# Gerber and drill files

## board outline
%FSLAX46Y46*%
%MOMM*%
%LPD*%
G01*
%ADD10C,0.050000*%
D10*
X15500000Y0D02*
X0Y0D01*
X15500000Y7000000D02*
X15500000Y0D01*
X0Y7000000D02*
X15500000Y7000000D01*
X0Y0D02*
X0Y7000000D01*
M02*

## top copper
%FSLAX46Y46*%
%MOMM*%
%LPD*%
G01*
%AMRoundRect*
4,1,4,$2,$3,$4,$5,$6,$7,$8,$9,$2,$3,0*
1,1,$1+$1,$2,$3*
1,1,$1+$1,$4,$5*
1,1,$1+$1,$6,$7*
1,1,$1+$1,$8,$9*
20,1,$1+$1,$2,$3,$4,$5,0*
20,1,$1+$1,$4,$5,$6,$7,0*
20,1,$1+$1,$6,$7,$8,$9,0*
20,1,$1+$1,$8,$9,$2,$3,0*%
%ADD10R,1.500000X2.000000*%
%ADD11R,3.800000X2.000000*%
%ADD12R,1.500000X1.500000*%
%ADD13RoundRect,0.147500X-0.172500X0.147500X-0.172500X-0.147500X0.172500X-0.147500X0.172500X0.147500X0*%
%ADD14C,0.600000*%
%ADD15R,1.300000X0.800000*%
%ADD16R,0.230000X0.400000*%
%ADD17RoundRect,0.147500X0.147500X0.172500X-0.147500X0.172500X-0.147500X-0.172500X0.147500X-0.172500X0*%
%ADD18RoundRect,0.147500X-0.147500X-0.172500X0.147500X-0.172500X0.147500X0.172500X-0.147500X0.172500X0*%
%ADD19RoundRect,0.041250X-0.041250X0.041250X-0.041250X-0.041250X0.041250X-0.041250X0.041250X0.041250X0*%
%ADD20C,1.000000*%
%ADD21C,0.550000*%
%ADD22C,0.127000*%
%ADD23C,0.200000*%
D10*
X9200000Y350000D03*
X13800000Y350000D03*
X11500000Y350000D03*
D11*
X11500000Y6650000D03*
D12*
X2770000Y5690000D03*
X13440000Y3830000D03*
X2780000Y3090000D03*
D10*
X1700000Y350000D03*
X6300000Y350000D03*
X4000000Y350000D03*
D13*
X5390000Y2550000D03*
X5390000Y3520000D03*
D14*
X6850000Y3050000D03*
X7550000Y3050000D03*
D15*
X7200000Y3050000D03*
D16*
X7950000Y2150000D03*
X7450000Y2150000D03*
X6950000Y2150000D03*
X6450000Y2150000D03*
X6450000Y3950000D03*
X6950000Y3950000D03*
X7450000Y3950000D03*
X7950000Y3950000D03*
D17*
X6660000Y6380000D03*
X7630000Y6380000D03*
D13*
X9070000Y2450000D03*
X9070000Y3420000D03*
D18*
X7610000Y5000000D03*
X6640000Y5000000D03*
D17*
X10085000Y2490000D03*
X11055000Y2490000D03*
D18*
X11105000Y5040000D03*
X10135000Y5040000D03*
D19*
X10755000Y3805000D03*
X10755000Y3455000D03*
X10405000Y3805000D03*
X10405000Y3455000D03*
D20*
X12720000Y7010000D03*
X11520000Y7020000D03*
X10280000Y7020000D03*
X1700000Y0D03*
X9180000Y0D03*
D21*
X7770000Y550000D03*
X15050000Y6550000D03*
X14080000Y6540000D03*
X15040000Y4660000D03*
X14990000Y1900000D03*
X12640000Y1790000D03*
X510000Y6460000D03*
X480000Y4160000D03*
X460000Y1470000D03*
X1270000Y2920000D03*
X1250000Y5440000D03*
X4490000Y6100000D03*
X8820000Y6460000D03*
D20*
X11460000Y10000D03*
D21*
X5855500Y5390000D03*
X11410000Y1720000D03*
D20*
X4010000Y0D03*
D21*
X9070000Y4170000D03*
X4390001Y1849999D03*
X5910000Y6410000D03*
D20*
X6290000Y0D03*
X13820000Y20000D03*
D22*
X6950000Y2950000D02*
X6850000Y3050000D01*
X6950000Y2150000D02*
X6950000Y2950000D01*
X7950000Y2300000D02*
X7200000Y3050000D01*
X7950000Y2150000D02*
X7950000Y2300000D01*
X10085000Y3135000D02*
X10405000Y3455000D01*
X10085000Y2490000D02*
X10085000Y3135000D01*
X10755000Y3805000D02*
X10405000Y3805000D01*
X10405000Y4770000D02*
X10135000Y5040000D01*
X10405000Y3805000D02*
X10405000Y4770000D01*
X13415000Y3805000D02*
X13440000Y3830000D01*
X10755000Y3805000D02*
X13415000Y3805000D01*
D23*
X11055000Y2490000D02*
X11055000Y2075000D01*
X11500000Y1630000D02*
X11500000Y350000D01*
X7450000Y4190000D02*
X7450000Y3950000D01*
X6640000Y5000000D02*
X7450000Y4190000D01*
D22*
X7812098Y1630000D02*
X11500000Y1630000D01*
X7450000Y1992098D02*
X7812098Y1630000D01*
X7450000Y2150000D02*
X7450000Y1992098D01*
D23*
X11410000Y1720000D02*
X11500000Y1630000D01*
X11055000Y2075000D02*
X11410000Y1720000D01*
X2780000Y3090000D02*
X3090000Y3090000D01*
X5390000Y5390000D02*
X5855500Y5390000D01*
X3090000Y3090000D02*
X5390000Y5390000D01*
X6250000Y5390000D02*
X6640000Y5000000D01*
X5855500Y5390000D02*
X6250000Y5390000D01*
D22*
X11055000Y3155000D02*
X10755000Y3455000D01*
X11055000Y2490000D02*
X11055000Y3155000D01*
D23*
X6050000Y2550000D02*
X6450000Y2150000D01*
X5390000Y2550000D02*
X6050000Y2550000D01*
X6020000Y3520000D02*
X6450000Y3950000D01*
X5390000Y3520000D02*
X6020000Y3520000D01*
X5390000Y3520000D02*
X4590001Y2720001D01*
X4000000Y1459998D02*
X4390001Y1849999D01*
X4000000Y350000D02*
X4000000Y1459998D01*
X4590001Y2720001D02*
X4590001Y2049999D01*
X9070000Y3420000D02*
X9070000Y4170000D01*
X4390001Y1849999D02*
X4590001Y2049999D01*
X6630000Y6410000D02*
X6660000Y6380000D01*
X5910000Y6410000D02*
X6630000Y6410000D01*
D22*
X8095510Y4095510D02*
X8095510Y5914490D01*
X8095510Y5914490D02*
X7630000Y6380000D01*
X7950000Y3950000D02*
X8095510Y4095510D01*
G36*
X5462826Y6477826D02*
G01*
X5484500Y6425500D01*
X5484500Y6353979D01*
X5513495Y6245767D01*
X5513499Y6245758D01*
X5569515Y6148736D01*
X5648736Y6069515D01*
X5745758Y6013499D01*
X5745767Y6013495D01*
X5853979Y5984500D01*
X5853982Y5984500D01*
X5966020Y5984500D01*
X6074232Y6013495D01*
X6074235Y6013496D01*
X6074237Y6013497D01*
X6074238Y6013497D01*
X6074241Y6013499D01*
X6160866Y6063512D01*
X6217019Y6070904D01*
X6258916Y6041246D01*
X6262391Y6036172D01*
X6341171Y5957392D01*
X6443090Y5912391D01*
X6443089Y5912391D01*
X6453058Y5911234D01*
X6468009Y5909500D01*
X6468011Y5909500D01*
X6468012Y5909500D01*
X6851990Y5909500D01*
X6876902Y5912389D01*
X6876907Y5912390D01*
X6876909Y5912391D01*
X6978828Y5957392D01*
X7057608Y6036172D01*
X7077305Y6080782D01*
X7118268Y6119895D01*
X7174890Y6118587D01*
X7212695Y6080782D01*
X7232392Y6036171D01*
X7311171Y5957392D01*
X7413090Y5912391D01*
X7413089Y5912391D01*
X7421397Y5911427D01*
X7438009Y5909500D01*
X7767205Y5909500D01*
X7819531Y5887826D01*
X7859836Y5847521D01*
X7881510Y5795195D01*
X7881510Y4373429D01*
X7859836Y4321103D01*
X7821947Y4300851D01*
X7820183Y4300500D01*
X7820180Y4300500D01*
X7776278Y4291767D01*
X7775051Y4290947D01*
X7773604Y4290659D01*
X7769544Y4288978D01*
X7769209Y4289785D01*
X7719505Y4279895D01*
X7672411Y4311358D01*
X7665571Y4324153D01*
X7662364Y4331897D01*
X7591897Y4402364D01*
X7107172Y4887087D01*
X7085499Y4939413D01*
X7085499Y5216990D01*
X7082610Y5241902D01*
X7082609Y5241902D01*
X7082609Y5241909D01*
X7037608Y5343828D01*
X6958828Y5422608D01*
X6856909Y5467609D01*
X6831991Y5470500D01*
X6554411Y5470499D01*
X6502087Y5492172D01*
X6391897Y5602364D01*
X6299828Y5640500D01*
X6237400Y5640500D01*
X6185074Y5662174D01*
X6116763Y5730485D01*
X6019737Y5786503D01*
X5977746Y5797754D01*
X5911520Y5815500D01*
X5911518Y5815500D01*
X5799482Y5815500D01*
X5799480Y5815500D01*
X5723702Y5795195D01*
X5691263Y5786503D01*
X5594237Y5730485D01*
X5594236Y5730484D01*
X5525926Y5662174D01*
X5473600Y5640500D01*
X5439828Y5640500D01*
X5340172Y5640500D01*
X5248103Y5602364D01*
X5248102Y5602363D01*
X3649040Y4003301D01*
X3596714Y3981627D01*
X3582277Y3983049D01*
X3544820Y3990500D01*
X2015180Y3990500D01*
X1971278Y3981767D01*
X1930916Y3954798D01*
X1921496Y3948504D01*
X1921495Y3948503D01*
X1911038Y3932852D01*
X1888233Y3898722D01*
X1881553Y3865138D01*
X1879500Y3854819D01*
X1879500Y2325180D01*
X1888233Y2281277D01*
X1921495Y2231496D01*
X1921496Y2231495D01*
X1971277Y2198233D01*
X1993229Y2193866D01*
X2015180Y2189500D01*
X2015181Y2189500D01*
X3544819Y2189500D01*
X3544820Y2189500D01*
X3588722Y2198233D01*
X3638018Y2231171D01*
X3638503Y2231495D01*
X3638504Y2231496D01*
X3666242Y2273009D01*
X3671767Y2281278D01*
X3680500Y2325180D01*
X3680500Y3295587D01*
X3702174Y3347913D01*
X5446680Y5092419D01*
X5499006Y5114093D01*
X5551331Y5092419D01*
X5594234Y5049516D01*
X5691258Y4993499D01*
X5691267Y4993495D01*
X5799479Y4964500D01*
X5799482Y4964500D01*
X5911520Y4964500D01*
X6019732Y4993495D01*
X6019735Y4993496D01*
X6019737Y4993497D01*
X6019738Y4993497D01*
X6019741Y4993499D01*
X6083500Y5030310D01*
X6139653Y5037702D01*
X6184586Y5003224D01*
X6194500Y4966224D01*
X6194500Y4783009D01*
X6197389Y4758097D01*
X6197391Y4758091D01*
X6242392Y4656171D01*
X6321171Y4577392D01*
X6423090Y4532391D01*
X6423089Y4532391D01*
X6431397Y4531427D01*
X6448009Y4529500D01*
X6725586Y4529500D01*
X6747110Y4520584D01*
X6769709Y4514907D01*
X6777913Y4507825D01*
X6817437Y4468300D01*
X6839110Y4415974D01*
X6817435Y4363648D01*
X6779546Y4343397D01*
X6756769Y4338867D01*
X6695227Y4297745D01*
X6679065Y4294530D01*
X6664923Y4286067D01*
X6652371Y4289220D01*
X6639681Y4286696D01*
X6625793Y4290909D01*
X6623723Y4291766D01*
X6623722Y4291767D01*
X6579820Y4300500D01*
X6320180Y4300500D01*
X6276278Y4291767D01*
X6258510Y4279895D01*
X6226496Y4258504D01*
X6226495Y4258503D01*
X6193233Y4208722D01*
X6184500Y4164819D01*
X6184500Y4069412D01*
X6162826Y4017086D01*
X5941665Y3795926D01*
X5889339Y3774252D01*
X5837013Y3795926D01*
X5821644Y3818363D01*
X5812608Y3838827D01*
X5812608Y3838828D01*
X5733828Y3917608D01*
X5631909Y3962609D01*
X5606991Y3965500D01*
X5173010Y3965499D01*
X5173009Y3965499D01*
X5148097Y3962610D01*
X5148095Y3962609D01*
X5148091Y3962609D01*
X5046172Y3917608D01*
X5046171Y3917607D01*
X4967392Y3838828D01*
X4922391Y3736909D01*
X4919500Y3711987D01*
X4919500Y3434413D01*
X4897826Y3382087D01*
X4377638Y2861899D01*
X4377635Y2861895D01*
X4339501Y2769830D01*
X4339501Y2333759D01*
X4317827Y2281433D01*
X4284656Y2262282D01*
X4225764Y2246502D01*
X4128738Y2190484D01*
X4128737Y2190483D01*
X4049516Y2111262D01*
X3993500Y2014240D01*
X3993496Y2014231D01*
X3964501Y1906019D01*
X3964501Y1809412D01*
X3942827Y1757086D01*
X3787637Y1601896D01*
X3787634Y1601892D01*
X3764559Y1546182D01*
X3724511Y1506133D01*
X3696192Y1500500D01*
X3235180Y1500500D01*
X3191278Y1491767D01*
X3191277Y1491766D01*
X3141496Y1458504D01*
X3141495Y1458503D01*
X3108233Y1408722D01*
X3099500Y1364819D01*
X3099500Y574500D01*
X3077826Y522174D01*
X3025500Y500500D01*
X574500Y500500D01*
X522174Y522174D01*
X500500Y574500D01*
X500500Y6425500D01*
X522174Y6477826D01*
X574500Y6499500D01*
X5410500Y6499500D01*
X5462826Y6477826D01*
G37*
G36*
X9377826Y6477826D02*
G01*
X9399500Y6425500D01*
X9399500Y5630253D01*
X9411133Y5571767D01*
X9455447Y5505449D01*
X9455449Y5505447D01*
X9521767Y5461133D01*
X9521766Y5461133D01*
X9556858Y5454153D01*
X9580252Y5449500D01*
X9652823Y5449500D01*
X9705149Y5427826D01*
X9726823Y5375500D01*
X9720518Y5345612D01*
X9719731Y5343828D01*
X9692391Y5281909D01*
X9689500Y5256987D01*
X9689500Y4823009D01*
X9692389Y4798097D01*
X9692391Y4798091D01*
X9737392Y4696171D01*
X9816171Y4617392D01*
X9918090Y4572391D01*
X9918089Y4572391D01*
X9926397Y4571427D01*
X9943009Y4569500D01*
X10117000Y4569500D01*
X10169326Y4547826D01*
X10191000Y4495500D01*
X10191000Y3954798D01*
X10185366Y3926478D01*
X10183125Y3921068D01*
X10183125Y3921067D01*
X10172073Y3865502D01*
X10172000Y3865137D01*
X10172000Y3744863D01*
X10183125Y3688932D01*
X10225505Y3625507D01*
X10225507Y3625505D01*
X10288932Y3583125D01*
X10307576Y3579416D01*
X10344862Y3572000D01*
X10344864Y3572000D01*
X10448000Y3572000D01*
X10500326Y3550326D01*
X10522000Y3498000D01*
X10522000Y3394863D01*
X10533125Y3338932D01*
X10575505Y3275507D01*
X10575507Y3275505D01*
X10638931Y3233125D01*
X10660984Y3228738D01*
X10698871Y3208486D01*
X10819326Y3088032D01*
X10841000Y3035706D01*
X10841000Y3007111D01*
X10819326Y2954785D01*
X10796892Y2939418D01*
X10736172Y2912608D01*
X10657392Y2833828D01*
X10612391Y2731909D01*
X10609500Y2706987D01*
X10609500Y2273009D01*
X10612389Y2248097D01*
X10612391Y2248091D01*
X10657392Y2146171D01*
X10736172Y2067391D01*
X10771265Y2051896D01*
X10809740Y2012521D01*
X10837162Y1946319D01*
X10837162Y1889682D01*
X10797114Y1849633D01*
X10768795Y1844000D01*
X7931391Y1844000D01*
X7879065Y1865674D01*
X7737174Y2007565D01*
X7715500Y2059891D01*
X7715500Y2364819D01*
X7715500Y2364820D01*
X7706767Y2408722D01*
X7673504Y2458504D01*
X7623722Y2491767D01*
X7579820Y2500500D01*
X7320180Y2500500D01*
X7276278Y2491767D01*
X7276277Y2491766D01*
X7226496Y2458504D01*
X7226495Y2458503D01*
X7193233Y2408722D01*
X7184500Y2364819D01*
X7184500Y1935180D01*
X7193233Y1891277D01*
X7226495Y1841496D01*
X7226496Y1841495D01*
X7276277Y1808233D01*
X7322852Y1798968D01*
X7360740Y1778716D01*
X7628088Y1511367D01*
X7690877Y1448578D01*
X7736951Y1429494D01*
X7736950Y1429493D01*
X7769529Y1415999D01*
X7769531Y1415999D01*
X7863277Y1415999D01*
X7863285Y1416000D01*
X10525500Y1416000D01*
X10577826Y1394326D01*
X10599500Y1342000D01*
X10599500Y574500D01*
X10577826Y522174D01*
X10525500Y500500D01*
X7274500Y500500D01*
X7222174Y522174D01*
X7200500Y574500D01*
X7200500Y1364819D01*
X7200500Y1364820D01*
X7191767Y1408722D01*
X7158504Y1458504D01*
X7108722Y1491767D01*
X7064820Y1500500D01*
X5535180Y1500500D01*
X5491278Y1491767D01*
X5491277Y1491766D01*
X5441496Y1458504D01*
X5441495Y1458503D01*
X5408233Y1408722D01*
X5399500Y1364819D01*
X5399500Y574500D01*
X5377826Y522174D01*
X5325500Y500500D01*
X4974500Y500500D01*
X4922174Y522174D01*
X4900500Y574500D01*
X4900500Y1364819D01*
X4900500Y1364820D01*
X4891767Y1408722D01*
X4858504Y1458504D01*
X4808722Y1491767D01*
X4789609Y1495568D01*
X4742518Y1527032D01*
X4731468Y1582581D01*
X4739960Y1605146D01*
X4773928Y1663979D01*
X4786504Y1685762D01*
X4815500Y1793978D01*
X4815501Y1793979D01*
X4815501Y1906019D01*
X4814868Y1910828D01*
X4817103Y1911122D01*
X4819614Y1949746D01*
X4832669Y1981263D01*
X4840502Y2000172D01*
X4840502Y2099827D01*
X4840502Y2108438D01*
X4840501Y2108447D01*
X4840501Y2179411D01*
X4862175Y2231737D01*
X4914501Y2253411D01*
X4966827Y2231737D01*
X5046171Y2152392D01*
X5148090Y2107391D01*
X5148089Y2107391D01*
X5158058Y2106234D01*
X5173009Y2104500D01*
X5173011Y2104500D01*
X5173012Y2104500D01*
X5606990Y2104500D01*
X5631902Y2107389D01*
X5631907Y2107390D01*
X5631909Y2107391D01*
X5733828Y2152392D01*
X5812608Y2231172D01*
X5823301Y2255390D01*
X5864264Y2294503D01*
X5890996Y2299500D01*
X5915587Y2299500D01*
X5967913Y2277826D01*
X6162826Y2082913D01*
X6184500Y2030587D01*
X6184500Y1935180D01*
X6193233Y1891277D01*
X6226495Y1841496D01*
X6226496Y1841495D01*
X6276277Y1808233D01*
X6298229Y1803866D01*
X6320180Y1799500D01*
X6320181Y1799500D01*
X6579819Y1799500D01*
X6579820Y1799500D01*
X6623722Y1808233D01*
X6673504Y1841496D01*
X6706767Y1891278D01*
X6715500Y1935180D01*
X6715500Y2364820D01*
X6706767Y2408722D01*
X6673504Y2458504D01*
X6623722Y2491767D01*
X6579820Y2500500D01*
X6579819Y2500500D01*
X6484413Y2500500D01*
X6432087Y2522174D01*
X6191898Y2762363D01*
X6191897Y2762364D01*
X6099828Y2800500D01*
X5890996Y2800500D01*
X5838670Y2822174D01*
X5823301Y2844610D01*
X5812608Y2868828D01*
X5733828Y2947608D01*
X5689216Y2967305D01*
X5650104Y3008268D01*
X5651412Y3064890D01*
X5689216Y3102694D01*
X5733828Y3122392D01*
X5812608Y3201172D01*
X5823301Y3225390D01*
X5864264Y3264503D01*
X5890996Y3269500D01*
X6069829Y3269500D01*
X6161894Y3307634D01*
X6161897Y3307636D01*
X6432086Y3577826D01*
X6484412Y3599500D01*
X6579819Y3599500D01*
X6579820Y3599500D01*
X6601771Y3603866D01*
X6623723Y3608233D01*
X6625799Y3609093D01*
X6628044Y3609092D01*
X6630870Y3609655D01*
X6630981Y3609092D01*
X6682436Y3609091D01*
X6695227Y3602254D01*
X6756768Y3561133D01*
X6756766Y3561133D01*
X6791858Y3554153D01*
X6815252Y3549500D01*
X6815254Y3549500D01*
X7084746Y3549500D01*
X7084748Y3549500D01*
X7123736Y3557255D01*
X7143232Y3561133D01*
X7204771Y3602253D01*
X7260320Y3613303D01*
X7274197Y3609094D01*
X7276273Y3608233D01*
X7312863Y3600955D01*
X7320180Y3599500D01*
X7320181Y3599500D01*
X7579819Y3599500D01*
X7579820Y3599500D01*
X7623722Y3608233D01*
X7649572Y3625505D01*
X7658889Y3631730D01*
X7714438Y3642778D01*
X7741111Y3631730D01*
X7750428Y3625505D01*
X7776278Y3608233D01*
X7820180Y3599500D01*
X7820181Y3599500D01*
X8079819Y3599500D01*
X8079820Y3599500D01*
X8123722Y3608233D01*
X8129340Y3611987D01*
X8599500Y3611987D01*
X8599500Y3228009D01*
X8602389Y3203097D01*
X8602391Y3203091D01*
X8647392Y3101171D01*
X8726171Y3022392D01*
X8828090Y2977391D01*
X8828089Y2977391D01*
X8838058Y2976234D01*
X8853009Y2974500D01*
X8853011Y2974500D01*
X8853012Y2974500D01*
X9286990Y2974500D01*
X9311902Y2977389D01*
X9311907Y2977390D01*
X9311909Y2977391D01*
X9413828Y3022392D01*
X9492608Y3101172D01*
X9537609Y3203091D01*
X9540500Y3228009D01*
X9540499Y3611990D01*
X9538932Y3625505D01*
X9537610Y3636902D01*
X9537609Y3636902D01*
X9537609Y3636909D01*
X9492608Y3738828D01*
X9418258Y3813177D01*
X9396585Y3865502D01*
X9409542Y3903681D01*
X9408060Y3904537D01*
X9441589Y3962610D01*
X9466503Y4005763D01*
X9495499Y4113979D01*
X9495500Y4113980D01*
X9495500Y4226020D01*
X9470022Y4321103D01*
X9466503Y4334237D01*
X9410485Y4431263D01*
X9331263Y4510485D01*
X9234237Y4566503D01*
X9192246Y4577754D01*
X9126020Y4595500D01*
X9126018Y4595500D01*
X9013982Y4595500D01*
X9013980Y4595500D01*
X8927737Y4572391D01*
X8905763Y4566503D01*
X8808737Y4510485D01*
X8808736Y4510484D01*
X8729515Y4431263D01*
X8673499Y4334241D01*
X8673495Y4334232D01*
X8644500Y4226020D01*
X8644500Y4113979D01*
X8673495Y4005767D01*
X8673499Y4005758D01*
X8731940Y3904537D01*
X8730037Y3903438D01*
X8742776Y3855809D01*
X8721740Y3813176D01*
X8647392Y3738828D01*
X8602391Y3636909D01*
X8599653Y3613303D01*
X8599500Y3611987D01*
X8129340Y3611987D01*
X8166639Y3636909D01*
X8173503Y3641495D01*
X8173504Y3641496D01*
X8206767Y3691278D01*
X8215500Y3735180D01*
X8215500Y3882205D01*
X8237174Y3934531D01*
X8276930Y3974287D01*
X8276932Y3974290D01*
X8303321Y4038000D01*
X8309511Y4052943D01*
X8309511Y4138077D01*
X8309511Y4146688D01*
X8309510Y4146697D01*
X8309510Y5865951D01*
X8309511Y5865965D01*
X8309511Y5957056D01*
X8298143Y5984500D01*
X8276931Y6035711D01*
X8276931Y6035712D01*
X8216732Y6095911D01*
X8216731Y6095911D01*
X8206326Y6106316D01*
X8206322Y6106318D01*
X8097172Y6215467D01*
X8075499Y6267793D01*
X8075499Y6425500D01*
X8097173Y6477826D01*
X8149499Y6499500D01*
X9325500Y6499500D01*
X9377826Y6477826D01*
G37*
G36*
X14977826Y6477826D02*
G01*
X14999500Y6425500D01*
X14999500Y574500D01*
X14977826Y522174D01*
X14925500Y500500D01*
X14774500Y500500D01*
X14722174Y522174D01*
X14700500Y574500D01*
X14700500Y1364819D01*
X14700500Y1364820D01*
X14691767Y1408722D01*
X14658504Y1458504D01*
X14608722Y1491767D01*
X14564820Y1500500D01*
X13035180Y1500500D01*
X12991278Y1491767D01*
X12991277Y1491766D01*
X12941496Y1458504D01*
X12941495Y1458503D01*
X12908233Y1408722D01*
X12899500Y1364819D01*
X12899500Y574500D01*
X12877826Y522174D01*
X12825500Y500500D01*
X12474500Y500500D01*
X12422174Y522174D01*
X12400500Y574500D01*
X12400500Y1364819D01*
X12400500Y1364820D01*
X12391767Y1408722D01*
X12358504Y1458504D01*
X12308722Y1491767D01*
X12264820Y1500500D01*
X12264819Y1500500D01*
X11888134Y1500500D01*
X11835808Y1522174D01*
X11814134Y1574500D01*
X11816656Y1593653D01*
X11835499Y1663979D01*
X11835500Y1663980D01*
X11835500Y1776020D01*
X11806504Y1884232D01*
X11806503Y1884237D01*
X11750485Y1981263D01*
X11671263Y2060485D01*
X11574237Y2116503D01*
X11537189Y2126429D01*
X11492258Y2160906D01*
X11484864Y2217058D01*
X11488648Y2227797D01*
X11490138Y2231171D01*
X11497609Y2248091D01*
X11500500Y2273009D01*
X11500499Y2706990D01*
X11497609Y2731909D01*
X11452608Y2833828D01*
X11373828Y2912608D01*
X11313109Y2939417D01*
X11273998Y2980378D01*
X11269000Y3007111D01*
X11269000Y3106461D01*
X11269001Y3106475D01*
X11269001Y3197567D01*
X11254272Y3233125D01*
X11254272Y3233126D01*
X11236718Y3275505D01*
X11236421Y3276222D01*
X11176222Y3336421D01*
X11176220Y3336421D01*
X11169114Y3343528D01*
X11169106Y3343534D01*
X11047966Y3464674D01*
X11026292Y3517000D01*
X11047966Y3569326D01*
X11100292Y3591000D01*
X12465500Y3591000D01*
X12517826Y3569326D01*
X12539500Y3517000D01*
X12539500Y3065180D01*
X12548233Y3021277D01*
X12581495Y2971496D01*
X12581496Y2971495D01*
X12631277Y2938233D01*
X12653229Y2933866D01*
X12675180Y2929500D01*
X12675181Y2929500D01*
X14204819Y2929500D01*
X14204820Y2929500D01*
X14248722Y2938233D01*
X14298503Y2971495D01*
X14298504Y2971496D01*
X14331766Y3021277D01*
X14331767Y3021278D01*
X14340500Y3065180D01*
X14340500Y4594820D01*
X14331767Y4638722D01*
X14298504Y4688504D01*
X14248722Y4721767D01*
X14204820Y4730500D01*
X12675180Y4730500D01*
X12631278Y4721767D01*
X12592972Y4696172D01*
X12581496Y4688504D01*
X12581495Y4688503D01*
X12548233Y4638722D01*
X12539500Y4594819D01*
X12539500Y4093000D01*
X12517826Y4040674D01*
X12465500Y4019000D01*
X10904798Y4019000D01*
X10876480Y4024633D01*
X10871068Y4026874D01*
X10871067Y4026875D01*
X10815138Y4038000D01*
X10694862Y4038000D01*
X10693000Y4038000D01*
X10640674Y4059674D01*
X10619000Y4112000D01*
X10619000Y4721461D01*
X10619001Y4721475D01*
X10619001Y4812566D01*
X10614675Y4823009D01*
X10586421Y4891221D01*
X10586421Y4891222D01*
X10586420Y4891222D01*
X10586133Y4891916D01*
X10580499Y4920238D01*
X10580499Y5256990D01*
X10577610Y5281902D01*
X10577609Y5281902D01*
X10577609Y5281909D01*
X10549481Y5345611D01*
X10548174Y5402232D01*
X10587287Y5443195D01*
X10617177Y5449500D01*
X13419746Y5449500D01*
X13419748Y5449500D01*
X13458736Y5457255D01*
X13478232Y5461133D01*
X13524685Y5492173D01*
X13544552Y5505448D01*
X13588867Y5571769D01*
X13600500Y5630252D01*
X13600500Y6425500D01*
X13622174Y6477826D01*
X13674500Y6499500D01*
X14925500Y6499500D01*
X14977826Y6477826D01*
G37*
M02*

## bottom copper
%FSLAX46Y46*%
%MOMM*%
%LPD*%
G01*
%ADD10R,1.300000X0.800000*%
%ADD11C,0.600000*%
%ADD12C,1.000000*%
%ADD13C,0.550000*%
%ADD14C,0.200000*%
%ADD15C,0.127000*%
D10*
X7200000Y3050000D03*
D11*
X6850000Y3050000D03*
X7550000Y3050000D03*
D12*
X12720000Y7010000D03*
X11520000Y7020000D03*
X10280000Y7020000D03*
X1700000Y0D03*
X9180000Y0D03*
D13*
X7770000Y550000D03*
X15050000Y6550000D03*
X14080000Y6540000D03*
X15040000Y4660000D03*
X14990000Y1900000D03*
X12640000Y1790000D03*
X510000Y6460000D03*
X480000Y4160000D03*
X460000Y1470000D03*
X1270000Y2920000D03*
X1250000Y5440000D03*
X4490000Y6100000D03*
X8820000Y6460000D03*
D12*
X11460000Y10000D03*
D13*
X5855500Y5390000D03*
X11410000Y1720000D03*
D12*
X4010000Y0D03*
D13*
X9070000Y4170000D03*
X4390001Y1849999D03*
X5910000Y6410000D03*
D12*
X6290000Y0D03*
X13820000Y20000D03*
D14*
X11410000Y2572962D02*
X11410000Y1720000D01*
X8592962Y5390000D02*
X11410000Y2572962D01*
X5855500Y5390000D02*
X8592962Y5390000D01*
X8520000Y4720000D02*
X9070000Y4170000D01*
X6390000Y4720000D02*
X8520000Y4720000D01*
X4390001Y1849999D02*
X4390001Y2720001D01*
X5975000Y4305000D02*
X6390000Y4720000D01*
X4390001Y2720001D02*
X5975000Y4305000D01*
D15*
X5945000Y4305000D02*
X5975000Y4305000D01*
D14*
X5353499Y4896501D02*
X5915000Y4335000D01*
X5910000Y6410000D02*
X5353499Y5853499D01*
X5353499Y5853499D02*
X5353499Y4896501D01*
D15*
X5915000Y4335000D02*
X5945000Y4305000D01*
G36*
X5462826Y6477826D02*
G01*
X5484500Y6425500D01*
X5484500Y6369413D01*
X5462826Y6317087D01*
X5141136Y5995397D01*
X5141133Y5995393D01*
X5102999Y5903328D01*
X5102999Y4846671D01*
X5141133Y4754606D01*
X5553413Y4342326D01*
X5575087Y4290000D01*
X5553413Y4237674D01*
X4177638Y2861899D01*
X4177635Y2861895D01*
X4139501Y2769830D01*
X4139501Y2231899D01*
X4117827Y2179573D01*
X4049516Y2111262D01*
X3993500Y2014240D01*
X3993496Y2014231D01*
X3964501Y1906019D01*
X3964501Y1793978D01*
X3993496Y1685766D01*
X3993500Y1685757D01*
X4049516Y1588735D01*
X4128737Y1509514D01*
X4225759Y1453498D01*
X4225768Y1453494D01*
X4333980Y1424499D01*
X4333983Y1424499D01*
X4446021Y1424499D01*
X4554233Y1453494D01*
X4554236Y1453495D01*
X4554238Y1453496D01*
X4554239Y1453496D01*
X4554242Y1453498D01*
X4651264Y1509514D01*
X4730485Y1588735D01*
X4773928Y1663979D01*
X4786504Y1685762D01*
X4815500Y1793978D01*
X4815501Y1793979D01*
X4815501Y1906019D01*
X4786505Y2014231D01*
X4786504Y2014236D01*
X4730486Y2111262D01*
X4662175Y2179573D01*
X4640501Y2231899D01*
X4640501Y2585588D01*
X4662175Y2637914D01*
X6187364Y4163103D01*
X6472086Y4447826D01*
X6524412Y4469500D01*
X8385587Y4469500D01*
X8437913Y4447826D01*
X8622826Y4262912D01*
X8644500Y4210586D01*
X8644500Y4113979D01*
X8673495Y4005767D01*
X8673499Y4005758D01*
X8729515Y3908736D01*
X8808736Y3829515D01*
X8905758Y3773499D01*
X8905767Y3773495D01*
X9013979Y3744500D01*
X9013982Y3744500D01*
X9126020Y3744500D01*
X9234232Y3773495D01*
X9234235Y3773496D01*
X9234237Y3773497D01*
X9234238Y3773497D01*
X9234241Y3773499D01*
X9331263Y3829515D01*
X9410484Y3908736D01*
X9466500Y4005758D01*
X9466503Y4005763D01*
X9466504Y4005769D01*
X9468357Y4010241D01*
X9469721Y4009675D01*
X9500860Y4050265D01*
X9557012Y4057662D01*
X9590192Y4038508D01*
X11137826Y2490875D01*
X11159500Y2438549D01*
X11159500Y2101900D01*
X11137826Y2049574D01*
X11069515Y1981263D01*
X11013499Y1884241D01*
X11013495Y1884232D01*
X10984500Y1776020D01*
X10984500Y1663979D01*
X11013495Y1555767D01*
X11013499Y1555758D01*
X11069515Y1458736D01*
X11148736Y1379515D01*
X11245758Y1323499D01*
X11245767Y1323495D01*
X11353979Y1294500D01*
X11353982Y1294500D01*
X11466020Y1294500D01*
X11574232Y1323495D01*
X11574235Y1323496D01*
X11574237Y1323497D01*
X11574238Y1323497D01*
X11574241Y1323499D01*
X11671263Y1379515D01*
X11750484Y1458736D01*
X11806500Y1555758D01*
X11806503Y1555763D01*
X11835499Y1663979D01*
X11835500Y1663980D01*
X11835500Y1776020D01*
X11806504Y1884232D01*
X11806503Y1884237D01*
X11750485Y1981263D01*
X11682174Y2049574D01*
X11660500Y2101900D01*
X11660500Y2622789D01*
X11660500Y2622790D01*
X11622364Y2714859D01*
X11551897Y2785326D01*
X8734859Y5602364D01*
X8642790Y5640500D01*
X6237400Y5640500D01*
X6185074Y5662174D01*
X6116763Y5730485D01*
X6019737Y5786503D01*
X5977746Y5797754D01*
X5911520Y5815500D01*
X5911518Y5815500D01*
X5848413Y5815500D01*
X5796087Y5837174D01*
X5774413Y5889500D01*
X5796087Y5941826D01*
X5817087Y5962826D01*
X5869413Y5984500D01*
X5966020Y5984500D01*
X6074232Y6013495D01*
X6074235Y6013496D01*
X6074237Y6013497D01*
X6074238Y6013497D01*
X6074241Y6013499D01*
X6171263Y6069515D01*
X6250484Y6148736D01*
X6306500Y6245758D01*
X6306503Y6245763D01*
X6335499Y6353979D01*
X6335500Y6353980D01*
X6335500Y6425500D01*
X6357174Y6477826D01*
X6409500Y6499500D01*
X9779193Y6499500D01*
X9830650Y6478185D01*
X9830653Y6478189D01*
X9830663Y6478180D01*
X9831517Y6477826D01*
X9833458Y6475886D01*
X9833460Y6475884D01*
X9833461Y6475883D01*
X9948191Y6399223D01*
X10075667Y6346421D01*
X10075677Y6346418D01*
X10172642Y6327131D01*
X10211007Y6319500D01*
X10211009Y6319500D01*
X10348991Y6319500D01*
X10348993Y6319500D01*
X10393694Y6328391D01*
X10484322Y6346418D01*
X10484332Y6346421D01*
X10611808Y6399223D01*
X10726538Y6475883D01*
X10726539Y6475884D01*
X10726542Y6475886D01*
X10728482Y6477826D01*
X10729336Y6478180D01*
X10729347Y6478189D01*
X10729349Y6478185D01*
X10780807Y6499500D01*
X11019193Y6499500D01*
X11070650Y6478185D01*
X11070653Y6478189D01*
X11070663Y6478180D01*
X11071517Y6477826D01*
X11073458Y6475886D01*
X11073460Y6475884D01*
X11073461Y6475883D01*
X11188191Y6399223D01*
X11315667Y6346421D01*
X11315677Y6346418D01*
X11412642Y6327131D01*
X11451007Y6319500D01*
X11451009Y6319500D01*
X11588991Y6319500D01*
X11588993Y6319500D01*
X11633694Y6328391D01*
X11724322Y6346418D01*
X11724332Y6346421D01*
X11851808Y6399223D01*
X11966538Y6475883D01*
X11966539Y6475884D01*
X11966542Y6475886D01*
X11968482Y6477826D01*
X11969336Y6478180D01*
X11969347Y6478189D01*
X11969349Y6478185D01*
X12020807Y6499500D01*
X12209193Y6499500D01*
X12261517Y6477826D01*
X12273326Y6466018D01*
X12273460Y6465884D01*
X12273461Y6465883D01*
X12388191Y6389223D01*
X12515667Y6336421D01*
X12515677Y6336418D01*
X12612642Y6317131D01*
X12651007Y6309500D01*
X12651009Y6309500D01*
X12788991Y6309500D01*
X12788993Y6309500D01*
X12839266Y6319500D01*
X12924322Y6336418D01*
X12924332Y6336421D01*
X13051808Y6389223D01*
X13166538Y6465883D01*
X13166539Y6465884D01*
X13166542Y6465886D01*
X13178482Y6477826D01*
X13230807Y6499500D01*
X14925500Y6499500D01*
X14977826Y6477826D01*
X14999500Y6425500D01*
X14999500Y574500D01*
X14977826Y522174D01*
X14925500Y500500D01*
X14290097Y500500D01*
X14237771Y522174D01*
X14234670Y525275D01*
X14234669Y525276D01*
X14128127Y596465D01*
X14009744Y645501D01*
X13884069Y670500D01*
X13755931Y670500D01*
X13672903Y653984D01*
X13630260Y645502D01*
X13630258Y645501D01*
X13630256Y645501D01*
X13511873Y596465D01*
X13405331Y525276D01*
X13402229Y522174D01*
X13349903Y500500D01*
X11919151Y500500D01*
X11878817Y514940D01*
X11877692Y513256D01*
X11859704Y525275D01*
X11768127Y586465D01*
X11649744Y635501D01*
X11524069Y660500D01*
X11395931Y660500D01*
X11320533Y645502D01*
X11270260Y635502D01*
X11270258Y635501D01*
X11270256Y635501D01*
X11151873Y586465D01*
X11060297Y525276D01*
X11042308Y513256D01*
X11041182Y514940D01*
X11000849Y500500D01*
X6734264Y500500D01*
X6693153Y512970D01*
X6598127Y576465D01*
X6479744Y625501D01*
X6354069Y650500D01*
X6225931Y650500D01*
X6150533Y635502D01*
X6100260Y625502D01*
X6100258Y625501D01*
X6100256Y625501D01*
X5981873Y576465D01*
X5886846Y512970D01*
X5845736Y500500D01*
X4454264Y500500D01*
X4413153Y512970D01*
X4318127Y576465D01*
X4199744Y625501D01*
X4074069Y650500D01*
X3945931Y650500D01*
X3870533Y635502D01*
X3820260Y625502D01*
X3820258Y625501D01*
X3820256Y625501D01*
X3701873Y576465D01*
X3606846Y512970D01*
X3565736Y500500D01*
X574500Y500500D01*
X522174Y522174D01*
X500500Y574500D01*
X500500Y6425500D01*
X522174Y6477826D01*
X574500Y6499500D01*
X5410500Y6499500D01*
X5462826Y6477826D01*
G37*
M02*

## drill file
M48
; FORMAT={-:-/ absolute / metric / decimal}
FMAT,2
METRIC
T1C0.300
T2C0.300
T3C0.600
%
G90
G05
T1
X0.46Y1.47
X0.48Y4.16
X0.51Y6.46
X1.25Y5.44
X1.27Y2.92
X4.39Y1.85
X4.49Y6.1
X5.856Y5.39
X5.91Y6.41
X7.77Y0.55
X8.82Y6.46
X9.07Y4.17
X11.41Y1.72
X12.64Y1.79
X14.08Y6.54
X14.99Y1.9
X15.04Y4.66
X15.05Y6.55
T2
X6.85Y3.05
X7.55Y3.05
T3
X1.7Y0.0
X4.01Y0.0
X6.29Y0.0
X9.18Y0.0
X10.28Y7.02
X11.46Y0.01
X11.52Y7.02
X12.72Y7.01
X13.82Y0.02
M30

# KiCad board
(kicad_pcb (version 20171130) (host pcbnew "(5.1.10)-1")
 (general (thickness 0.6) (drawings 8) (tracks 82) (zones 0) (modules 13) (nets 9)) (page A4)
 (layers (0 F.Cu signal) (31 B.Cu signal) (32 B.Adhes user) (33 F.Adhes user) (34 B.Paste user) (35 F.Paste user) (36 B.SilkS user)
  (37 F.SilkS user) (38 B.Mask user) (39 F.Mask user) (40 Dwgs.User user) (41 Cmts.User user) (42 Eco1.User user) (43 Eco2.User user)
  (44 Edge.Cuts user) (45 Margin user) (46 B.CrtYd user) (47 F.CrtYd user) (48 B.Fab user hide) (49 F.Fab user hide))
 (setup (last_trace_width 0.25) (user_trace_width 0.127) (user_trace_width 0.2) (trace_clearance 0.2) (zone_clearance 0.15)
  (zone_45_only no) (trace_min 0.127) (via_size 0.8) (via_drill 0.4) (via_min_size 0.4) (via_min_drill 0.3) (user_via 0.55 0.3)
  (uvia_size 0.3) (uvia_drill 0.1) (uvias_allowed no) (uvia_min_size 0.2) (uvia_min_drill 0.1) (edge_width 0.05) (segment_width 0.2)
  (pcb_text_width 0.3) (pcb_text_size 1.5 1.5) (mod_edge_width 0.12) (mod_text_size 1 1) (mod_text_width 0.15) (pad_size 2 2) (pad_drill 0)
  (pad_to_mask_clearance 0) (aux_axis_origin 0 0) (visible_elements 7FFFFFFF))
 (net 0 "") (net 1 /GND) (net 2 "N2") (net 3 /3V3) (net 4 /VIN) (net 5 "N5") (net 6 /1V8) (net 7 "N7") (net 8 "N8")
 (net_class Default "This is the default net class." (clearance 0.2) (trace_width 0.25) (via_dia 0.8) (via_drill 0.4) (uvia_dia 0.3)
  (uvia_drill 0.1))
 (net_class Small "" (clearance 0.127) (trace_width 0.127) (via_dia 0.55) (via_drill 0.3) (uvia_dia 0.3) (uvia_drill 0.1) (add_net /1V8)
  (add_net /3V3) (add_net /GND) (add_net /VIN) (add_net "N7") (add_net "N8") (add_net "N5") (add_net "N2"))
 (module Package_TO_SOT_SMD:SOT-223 (layer F.Cu) (at 11.5 -3.5 90)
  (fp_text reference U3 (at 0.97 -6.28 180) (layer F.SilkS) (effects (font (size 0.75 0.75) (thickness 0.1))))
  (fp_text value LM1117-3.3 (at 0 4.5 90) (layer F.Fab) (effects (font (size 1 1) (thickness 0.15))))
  (pad 1 smd rect (at -3.15 -2.3 90) (size 2 1.5) (layers F.Cu F.Paste F.Mask) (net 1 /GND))
  (pad 3 smd rect (at -3.15 2.3 90) (size 2 1.5) (layers F.Cu F.Paste F.Mask) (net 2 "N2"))
  (pad 2 smd rect (at -3.15 0 90) (size 2 1.5) (layers F.Cu F.Paste F.Mask) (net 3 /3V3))
  (pad 4 smd rect (at 3.15 0 90) (size 2 3.8) (layers F.Cu F.Paste F.Mask)))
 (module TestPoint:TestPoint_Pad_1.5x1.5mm (layer F.Cu) (at 2.77 -5.69)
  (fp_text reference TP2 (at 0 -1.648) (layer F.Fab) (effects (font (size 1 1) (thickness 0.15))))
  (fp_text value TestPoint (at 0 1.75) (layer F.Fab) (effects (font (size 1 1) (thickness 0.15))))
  (pad 1 smd rect (at 0 0) (size 1.5 1.5) (layers F.Cu F.Mask) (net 1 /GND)))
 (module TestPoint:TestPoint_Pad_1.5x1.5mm (layer F.Cu) (at 13.44 -3.83)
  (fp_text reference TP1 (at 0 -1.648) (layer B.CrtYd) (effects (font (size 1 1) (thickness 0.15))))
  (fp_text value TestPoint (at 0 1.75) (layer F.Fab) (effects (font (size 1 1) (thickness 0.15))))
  (pad 1 smd rect (at 0 0) (size 1.5 1.5) (layers F.Cu F.Mask) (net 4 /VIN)))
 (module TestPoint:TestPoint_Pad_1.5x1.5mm (layer F.Cu) (at 2.78 -3.09)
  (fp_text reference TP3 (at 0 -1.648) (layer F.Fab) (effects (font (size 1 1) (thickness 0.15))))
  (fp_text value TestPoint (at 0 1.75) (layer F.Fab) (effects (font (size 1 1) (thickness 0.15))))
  (pad 1 smd rect (at 0 0) (size 1.5 1.5) (layers F.Cu F.Mask) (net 3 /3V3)))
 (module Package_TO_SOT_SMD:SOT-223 (layer F.Cu) (at 4 -3.5 90)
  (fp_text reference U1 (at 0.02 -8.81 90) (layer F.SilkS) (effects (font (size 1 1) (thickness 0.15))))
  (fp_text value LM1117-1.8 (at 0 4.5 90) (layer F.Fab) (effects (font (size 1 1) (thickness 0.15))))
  (pad 1 smd rect (at -3.15 -2.3 90) (size 2 1.5) (layers F.Cu F.Paste F.Mask) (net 1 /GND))
  (pad 3 smd rect (at -3.15 2.3 90) (size 2 1.5) (layers F.Cu F.Paste F.Mask) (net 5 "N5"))
  (pad 2 smd rect (at -3.15 0 90) (size 2 1.5) (layers F.Cu F.Paste F.Mask) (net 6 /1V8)))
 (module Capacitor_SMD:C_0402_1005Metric (layer F.Cu) (at 5.39 -3.035 270)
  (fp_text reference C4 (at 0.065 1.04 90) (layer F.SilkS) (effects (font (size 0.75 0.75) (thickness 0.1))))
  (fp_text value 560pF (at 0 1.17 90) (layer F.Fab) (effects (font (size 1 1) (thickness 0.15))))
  (pad 2 smd roundrect (at 0.485 0 270) (size 0.59 0.64) (layers F.Cu F.Paste F.Mask) (roundrect_rratio 0.25) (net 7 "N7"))
  (pad 1 smd roundrect (at -0.485 0 270) (size 0.59 0.64) (layers F.Cu F.Paste F.Mask) (roundrect_rratio 0.25) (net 6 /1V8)))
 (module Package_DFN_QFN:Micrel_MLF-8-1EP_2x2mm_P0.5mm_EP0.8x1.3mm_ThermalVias (layer F.Cu) (at 7.2 -3.05 270)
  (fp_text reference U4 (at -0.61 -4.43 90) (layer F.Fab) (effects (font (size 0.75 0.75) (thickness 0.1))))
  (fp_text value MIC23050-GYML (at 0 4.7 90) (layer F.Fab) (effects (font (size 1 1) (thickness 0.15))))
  (pad 9 smd rect (at 0 0 270) (size 0.8 1.3) (layers B.Cu) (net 1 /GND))
  (pad "" smd rect (at 0 0.35 270) (size 0.55 0.55) (layers F.Paste))
  (pad "" smd rect (at 0 -0.35 270) (size 0.55 0.55) (layers F.Paste))
  (pad 9 thru_hole circle (at 0 0.35 270) (size 0.6 0.6) (drill 0.3) (layers *.Cu) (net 1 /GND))
  (pad 9 thru_hole circle (at 0 -0.35 270) (size 0.6 0.6) (drill 0.3) (layers *.Cu) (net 1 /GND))
  (pad 9 smd rect (at 0 0 270) (size 0.8 1.3) (layers F.Cu F.Mask) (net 1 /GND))
  (pad 8 smd rect (at 0.9 -0.75 270) (size 0.4 0.23) (layers F.Cu F.Paste F.Mask) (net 1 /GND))
  (pad 7 smd rect (at 0.9 -0.25 270) (size 0.4 0.23) (layers F.Cu F.Paste F.Mask) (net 3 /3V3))
  (pad 6 smd rect (at 0.9 0.25 270) (size 0.4 0.23) (layers F.Cu F.Paste F.Mask) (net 1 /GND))
  (pad 5 smd rect (at 0.9 0.75 270) (size 0.4 0.23) (layers F.Cu F.Paste F.Mask) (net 7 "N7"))
  (pad 4 smd rect (at -0.9 0.75 270) (size 0.4 0.23) (layers F.Cu F.Paste F.Mask) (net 6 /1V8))
  (pad 3 smd rect (at -0.9 0.25 270) (size 0.4 0.23) (layers F.Cu F.Paste F.Mask))
  (pad 2 smd rect (at -0.9 -0.25 270) (size 0.4 0.23) (layers F.Cu F.Paste F.Mask) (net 3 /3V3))
  (pad 1 smd rect (at -0.9 -0.75 270) (size 0.4 0.23) (layers F.Cu F.Paste F.Mask) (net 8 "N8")))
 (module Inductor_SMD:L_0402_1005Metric (layer F.Cu) (at 7.145 -6.38 180)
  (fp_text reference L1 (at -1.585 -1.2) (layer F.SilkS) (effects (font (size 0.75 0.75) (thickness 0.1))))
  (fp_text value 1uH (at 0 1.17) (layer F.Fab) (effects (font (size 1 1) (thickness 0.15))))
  (pad 2 smd roundrect (at 0.485 0 180) (size 0.59 0.64) (layers F.Cu F.Paste F.Mask) (roundrect_rratio 0.25) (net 6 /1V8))
  (pad 1 smd roundrect (at -0.485 0 180) (size 0.59 0.64) (layers F.Cu F.Paste F.Mask) (roundrect_rratio 0.25) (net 8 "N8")))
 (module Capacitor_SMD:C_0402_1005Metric (layer F.Cu) (at 9.07 -2.935 270)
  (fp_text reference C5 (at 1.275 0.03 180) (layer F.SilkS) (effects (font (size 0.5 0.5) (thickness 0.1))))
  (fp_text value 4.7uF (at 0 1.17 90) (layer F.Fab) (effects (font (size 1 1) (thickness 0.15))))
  (pad 2 smd roundrect (at 0.485 0 270) (size 0.59 0.64) (layers F.Cu F.Paste F.Mask) (roundrect_rratio 0.25) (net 1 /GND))
  (pad 1 smd roundrect (at -0.485 0 270) (size 0.59 0.64) (layers F.Cu F.Paste F.Mask) (roundrect_rratio 0.25) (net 6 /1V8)))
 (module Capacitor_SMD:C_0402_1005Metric (layer F.Cu) (at 7.125 -5)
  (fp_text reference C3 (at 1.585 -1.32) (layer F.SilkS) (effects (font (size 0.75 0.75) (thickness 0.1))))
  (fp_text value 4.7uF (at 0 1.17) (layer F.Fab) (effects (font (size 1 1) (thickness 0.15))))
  (pad 2 smd roundrect (at 0.485 0) (size 0.59 0.64) (layers F.Cu F.Paste F.Mask) (roundrect_rratio 0.25) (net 1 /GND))
  (pad 1 smd roundrect (at -0.485 0) (size 0.59 0.64) (layers F.Cu F.Paste F.Mask) (roundrect_rratio 0.25) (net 3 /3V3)))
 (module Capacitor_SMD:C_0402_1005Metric (layer F.Cu) (at 10.57 -2.49 180)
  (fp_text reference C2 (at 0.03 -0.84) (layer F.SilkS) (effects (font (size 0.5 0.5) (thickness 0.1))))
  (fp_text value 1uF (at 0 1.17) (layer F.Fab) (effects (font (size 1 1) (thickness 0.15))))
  (pad 2 smd roundrect (at 0.485 0 180) (size 0.59 0.64) (layers F.Cu F.Paste F.Mask) (roundrect_rratio 0.25) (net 1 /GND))
  (pad 1 smd roundrect (at -0.485 0 180) (size 0.59 0.64) (layers F.Cu F.Paste F.Mask) (roundrect_rratio 0.25) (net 3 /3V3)))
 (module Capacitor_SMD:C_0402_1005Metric (layer F.Cu) (at 10.62 -5.04)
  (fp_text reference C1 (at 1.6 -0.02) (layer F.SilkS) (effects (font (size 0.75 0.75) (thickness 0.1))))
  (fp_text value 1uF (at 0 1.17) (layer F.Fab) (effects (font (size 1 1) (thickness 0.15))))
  (pad 2 smd roundrect (at 0.485 0) (size 0.59 0.64) (layers F.Cu F.Paste F.Mask) (roundrect_rratio 0.25) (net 1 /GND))
  (pad 1 smd roundrect (at -0.485 0) (size 0.59 0.64) (layers F.Cu F.Paste F.Mask) (roundrect_rratio 0.25) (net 4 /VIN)))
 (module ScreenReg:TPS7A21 (layer F.Cu) (at 10.58 -3.63 270)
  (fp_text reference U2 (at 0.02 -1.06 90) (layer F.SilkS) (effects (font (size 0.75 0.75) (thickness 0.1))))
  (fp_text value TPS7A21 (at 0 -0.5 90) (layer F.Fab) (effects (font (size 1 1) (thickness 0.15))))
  (pad A1 smd roundrect (at -0.175 -0.175 270) (size 0.165 0.165) (layers F.Cu F.Paste F.Mask) (roundrect_rratio 0.25) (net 4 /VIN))
  (pad A2 smd roundrect (at 0.175 -0.175 270) (size 0.165 0.165) (layers F.Cu F.Paste F.Mask) (roundrect_rratio 0.25) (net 3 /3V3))
  (pad B1 smd roundrect (at -0.175 0.175 270) (size 0.165 0.165) (layers F.Cu F.Paste F.Mask) (roundrect_rratio 0.25) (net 4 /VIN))
  (pad B2 smd roundrect (at 0.175 0.175 270) (size 0.165 0.165) (layers F.Cu F.Paste F.Mask) (roundrect_rratio 0.25) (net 1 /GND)))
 (gr_line (start 15.5 0) (end 0 0) (layer Edge.Cuts) (width 0.05))
 (gr_line (start 15.5 -7) (end 15.5 0) (layer Edge.Cuts) (width 0.05))
 (gr_line (start 0 -7) (end 15.5 -7) (layer Edge.Cuts) (width 0.05))
 (gr_line (start 0 0) (end 0 -7) (layer Edge.Cuts) (width 0.05))
 (via (at 12.72 -7.01) (size 1) (drill 0.6) (layers F.Cu B.Cu) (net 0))
 (via (at 11.52 -7.02) (size 1) (drill 0.6) (layers F.Cu B.Cu) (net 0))
 (via (at 10.28 -7.02) (size 1) (drill 0.6) (layers F.Cu B.Cu) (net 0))
 (via (at 1.7 0) (size 1) (drill 0.6) (layers F.Cu B.Cu) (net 1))
 (via (at 9.18 0) (size 1) (drill 0.6) (layers F.Cu B.Cu) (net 1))
 (via (at 7.77 -0.55) (size 0.55) (drill 0.3) (layers F.Cu B.Cu) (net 1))
 (segment (start 6.95 -2.95) (end 6.85 -3.05) (width 0.127) (layer F.Cu) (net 1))
 (segment (start 6.95 -2.15) (end 6.95 -2.95) (width 0.127) (layer F.Cu) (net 1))
 (segment (start 7.95 -2.3) (end 7.2 -3.05) (width 0.127) (layer F.Cu) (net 1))
 (segment (start 7.95 -2.15) (end 7.95 -2.3) (width 0.127) (layer F.Cu) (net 1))
 (via (at 15.05 -6.55) (size 0.55) (drill 0.3) (layers F.Cu B.Cu) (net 1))
 (via (at 14.08 -6.54) (size 0.55) (drill 0.3) (layers F.Cu B.Cu) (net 1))
 (via (at 15.04 -4.66) (size 0.55) (drill 0.3) (layers F.Cu B.Cu) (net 1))
 (via (at 14.99 -1.9) (size 0.55) (drill 0.3) (layers F.Cu B.Cu) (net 1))
 (via (at 12.64 -1.79) (size 0.55) (drill 0.3) (layers F.Cu B.Cu) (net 1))
 (via (at 0.51 -6.46) (size 0.55) (drill 0.3) (layers F.Cu B.Cu) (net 1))
 (via (at 0.48 -4.16) (size 0.55) (drill 0.3) (layers F.Cu B.Cu) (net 1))
 (via (at 0.46 -1.47) (size 0.55) (drill 0.3) (layers F.Cu B.Cu) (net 1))
 (via (at 1.27 -2.92) (size 0.55) (drill 0.3) (layers F.Cu B.Cu) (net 1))
 (via (at 1.25 -5.44) (size 0.55) (drill 0.3) (layers F.Cu B.Cu) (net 1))
 (via (at 4.49 -6.1) (size 0.55) (drill 0.3) (layers F.Cu B.Cu) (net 1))
 (via (at 8.82 -6.46) (size 0.55) (drill 0.3) (layers F.Cu B.Cu) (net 1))
 (segment (start 10.085 -3.135) (end 10.405 -3.455) (width 0.127) (layer F.Cu) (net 1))
 (segment (start 10.085 -2.49) (end 10.085 -3.135) (width 0.127) (layer F.Cu) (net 1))
 (segment (start 10.755 -3.805) (end 10.405 -3.805) (width 0.127) (layer F.Cu) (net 4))
 (segment (start 10.405 -4.77) (end 10.135 -5.04) (width 0.127) (layer F.Cu) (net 4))
 (segment (start 10.405 -3.805) (end 10.405 -4.77) (width 0.127) (layer F.Cu) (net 4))
 (segment (start 13.415 -3.805) (end 13.44 -3.83) (width 0.127) (layer F.Cu) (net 4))
 (segment (start 10.755 -3.805) (end 13.415 -3.805) (width 0.127) (layer F.Cu) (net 4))
 (via (at 11.46 -0.01) (size 1) (drill 0.6) (layers F.Cu B.Cu) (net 3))
 (segment (start 11.055 -2.49) (end 11.055 -2.075) (width 0.2) (layer F.Cu) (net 3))
 (segment (start 11.5 -1.63) (end 11.5 -0.35) (width 0.2) (layer F.Cu) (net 3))
 (segment (start 7.45 -4.19) (end 7.45 -3.95) (width 0.2) (layer F.Cu) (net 3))
 (segment (start 6.64 -5) (end 7.45 -4.19) (width 0.2) (layer F.Cu) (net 3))
 (segment (start 7.812098 -1.63) (end 11.5 -1.63) (width 0.127) (layer F.Cu) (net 3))
 (segment (start 7.45 -1.992098) (end 7.812098 -1.63) (width 0.127) (layer F.Cu) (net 3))
 (segment (start 7.45 -2.15) (end 7.45 -1.992098) (width 0.127) (layer F.Cu) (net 3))
 (via (at 5.8555 -5.39) (size 0.55) (drill 0.3) (layers F.Cu B.Cu) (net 3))
 (via (at 11.41 -1.72) (size 0.55) (drill 0.3) (layers F.Cu B.Cu) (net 3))
 (segment (start 11.41 -1.72) (end 11.5 -1.63) (width 0.2) (layer F.Cu) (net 3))
 (segment (start 11.055 -2.075) (end 11.41 -1.72) (width 0.2) (layer F.Cu) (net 3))
 (segment (start 2.78 -3.09) (end 3.09 -3.09) (width 0.2) (layer F.Cu) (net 3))
 (segment (start 5.39 -5.39) (end 5.8555 -5.39) (width 0.2) (layer F.Cu) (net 3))
 (segment (start 3.09 -3.09) (end 5.39 -5.39) (width 0.2) (layer F.Cu) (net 3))
 (segment (start 6.25 -5.39) (end 6.64 -5) (width 0.2) (layer F.Cu) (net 3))
 (segment (start 5.8555 -5.39) (end 6.25 -5.39) (width 0.2) (layer F.Cu) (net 3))
 (segment (start 11.41 -2.572962) (end 11.41 -1.72) (width 0.2) (layer B.Cu) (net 3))
 (segment (start 8.592962 -5.39) (end 11.41 -2.572962) (width 0.2) (layer B.Cu) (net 3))
 (segment (start 5.8555 -5.39) (end 8.592962 -5.39) (width 0.2) (layer B.Cu) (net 3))
 (segment (start 11.055 -3.155) (end 10.755 -3.455) (width 0.127) (layer F.Cu) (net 3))
 (segment (start 11.055 -2.49) (end 11.055 -3.155) (width 0.127) (layer F.Cu) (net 3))
 (segment (start 6.05 -2.55) (end 6.45 -2.15) (width 0.2) (layer F.Cu) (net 7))
 (segment (start 5.39 -2.55) (end 6.05 -2.55) (width 0.2) (layer F.Cu) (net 7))
 (via (at 4.01 0) (size 1) (drill 0.6) (layers F.Cu B.Cu) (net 6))
 (via (at 9.07 -4.17) (size 0.55) (drill 0.3) (layers F.Cu B.Cu) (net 6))
 (segment (start 6.02 -3.52) (end 6.45 -3.95) (width 0.2) (layer F.Cu) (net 6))
 (segment (start 5.39 -3.52) (end 6.02 -3.52) (width 0.2) (layer F.Cu) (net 6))
 (segment (start 5.39 -3.52) (end 4.590001 -2.720001) (width 0.2) (layer F.Cu) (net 6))
 (segment (start 4 -1.459998) (end 4.390001 -1.849999) (width 0.2) (layer F.Cu) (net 6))
 (segment (start 4 -0.35) (end 4 -1.459998) (width 0.2) (layer F.Cu) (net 6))
 (segment (start 4.590001 -2.720001) (end 4.590001 -2.049999) (width 0.2) (layer F.Cu) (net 6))
 (segment (start 9.07 -3.42) (end 9.07 -4.17) (width 0.2) (layer F.Cu) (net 6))
 (segment (start 4.390001 -1.849999) (end 4.590001 -2.049999) (width 0.2) (layer F.Cu) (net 6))
 (via (at 4.390001 -1.849999) (size 0.55) (drill 0.3) (layers F.Cu B.Cu) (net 6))
 (segment (start 8.52 -4.72) (end 9.07 -4.17) (width 0.2) (layer B.Cu) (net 6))
 (segment (start 6.39 -4.72) (end 8.52 -4.72) (width 0.2) (layer B.Cu) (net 6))
 (segment (start 4.390001 -1.849999) (end 4.390001 -2.720001) (width 0.2) (layer B.Cu) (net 6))
 (via (at 5.91 -6.41) (size 0.55) (drill 0.3) (layers F.Cu B.Cu) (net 6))
 (segment (start 5.975 -4.305) (end 6.39 -4.72) (width 0.2) (layer B.Cu) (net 6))
 (segment (start 4.390001 -2.720001) (end 5.975 -4.305) (width 0.2) (layer B.Cu) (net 6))
 (segment (start 5.945 -4.305) (end 5.975 -4.305) (width 0.127) (layer B.Cu) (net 6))
 (segment (start 6.63 -6.41) (end 6.66 -6.38) (width 0.2) (layer F.Cu) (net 6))
 (segment (start 5.91 -6.41) (end 6.63 -6.41) (width 0.2) (layer F.Cu) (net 6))
 (segment (start 5.353499 -4.896501) (end 5.915 -4.335) (width 0.2) (layer B.Cu) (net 6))
 (segment (start 5.91 -6.41) (end 5.353499 -5.853499) (width 0.2) (layer B.Cu) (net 6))
 (segment (start 5.353499 -5.853499) (end 5.353499 -4.896501) (width 0.2) (layer B.Cu) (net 6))
 (segment (start 5.915 -4.335) (end 5.945 -4.305) (width 0.127) (layer B.Cu) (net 6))
 (segment (start 8.09551 -4.09551) (end 8.09551 -5.91449) (width 0.127) (layer F.Cu) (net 8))
 (segment (start 8.09551 -5.91449) (end 7.63 -6.38) (width 0.127) (layer F.Cu) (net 8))
 (segment (start 7.95 -3.95) (end 8.09551 -4.09551) (width 0.127) (layer F.Cu) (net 8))
 (via (at 6.29 0) (size 1) (drill 0.6) (layers F.Cu B.Cu) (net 5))
 (via (at 13.82 -0.02) (size 1) (drill 0.6) (layers F.Cu B.Cu) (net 2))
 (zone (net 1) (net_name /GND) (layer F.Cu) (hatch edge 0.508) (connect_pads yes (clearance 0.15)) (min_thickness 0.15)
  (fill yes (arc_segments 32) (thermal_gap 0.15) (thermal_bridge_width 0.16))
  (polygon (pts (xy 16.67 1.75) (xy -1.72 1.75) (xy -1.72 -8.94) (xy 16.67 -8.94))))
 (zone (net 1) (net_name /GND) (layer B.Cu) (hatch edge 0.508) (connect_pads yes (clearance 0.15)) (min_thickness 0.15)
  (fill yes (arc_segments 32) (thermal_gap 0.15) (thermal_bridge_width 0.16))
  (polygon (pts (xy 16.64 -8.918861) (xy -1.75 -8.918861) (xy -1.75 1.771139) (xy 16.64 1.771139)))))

